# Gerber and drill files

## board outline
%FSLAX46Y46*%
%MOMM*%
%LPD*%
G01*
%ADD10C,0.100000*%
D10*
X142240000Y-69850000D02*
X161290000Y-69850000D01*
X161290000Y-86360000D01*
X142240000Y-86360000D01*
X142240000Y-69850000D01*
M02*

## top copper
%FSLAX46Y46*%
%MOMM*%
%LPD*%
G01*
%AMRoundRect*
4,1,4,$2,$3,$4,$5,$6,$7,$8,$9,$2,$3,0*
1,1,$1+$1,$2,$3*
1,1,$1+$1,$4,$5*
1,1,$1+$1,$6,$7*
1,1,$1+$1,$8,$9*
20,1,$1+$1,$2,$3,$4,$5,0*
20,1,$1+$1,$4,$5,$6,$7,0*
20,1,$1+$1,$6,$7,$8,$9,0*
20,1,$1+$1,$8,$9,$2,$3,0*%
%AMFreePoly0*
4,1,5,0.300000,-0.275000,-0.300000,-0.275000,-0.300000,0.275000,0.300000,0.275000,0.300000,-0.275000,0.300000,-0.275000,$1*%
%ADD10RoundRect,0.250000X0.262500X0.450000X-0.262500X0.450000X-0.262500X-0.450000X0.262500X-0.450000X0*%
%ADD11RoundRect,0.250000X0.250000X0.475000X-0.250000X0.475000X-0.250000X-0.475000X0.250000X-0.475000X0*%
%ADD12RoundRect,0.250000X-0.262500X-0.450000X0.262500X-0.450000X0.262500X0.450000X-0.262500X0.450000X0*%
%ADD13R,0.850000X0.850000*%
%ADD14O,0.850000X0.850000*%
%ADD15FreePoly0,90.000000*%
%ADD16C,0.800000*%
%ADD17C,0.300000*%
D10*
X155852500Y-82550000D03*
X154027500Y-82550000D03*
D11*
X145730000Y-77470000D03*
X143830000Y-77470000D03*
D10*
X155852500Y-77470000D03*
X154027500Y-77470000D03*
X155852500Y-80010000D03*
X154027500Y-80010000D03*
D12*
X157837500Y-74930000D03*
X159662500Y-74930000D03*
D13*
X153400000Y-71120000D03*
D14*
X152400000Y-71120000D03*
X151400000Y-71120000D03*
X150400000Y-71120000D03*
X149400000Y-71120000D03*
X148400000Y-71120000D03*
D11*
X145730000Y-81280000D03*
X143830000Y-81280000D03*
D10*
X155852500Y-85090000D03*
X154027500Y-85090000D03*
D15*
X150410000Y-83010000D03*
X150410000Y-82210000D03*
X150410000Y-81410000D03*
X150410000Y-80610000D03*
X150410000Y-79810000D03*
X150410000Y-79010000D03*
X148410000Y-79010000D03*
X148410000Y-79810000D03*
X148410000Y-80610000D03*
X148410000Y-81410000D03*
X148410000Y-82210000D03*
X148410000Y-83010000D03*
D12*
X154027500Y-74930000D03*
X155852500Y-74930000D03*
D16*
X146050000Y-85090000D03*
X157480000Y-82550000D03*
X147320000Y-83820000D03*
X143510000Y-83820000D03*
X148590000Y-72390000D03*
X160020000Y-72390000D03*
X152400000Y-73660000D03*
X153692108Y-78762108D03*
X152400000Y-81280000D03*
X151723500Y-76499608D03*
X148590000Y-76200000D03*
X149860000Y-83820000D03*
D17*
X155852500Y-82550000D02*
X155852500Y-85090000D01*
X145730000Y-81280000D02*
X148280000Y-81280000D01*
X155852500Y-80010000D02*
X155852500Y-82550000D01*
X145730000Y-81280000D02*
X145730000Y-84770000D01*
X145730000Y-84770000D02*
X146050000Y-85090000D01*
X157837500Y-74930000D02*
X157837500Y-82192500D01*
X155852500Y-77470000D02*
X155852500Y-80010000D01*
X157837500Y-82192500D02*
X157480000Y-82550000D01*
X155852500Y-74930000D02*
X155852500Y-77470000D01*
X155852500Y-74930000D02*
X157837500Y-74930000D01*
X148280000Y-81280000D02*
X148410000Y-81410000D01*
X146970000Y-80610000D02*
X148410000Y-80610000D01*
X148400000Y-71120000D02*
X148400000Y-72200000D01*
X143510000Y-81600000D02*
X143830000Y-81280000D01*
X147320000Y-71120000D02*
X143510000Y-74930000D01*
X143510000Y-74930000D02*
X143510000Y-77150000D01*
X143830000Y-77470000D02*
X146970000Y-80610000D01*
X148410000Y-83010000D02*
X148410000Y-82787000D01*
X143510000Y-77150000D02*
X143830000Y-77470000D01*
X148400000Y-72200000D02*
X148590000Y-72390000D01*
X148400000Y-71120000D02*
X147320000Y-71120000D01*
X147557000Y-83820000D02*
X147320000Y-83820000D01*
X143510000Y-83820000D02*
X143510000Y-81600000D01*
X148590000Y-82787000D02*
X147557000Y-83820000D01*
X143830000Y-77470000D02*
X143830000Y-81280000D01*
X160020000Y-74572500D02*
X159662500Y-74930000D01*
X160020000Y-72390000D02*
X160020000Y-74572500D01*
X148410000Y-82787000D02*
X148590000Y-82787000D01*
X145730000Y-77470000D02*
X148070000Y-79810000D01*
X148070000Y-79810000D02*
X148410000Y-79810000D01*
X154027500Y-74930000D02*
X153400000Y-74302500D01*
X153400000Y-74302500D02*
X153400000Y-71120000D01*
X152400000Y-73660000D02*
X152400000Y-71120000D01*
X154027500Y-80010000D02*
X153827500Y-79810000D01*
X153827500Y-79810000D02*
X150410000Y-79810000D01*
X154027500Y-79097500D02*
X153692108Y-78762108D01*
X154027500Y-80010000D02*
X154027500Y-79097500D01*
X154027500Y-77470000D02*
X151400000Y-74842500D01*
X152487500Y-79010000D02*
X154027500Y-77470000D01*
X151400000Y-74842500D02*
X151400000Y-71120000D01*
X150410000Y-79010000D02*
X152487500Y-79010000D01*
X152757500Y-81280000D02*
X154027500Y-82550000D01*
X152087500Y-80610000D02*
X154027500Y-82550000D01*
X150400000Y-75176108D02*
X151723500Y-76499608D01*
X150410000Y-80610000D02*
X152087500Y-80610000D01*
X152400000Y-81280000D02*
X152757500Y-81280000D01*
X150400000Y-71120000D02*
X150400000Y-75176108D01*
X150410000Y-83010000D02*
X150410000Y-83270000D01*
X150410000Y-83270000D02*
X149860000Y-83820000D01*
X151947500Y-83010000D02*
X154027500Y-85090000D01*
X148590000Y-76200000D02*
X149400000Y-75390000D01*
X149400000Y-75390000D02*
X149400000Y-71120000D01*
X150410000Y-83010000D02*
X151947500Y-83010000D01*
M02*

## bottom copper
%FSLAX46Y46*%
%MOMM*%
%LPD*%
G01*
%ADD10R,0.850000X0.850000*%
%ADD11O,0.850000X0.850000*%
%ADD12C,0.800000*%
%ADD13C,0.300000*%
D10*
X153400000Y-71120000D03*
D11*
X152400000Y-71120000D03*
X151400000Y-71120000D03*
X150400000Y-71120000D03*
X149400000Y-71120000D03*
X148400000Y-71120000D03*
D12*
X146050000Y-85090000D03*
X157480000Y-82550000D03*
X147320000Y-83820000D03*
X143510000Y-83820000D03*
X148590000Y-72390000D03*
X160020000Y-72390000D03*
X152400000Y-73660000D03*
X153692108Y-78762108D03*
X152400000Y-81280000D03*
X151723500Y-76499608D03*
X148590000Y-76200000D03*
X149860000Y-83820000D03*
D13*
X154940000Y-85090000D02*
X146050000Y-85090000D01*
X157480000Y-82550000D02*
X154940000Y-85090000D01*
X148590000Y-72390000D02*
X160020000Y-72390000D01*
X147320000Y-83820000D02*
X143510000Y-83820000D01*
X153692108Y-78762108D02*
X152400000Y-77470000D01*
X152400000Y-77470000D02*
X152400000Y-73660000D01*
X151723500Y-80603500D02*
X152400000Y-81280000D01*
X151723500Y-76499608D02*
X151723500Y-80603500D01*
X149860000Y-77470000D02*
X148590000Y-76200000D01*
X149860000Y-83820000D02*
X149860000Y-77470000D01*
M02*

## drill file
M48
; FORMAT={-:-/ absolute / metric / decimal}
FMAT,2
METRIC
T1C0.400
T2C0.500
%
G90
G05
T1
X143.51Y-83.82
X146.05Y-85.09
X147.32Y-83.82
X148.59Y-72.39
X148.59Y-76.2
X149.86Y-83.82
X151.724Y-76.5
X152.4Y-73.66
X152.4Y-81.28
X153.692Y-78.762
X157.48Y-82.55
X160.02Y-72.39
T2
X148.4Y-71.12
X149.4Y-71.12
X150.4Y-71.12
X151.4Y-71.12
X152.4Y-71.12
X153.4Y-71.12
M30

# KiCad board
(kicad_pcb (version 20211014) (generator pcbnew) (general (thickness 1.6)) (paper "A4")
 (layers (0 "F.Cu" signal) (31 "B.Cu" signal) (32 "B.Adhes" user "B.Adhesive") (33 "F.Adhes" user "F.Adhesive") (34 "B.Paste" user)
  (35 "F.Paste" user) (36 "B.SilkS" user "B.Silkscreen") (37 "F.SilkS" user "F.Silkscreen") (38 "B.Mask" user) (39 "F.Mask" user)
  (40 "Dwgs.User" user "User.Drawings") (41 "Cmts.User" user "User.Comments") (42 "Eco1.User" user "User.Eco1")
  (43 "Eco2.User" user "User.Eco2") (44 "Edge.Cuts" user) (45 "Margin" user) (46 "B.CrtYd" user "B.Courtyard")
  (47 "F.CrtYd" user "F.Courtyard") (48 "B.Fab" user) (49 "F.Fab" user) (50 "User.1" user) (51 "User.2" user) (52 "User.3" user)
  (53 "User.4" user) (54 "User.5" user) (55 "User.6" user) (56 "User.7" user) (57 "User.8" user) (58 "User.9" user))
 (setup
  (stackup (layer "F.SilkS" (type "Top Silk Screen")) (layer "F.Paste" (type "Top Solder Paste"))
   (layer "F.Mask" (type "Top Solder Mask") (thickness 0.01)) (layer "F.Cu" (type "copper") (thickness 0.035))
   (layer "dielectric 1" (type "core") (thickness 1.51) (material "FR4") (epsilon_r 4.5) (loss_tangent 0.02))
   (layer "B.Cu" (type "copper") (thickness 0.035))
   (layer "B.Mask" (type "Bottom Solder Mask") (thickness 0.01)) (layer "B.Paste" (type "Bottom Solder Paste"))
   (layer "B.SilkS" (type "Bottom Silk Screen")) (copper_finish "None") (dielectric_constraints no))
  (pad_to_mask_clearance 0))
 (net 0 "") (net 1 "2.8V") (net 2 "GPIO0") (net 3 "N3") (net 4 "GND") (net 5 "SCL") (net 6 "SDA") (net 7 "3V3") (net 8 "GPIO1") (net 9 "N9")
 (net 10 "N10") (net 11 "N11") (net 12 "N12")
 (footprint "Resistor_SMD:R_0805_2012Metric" (layer "F.Cu") (at 154.94 82.55 180)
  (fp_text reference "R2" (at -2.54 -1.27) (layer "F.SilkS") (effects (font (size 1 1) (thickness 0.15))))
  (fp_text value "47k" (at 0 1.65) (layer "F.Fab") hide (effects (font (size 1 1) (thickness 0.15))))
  (pad "1" smd roundrect (at -0.9125 0 180) (size 1.025 1.4) (layers "F.Cu" "F.Paste" "F.Mask") (roundrect_rratio 0.243902) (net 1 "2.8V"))
  (pad "2" smd roundrect (at 0.9125 0 180) (size 1.025 1.4) (layers "F.Cu" "F.Paste" "F.Mask") (roundrect_rratio 0.243902) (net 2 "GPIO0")))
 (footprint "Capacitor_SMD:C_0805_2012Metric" (layer "F.Cu") (at 144.78 77.47 180)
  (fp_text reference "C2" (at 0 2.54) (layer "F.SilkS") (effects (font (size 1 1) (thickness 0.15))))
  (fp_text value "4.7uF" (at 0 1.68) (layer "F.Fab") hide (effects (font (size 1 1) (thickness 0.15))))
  (pad "1" smd roundrect (at -0.95 0 180) (size 1 1.45) (layers "F.Cu" "F.Paste" "F.Mask") (roundrect_rratio 0.25) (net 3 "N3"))
  (pad "2" smd roundrect (at 0.95 0 180) (size 1 1.45) (layers "F.Cu" "F.Paste" "F.Mask") (roundrect_rratio 0.25) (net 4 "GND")))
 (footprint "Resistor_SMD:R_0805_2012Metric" (layer "F.Cu") (at 154.94 77.47 180)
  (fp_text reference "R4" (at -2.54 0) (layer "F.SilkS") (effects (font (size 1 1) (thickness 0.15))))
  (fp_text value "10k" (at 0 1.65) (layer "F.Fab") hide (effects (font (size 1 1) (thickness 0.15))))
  (pad "1" smd roundrect (at -0.9125 0 180) (size 1.025 1.4) (layers "F.Cu" "F.Paste" "F.Mask") (roundrect_rratio 0.243902) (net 1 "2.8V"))
  (pad "2" smd roundrect (at 0.9125 0 180) (size 1.025 1.4) (layers "F.Cu" "F.Paste" "F.Mask") (roundrect_rratio 0.243902) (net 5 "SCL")))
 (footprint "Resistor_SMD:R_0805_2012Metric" (layer "F.Cu") (at 154.94 80.01 180)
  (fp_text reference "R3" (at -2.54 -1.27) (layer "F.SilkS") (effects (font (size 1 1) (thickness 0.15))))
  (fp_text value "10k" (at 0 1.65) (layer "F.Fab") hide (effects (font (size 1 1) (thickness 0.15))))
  (pad "1" smd roundrect (at -0.9125 0 180) (size 1.025 1.4) (layers "F.Cu" "F.Paste" "F.Mask") (roundrect_rratio 0.243902) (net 1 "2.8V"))
  (pad "2" smd roundrect (at 0.9125 0 180) (size 1.025 1.4) (layers "F.Cu" "F.Paste" "F.Mask") (roundrect_rratio 0.243902) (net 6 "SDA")))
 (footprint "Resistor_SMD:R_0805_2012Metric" (layer "F.Cu") (at 158.75 74.93)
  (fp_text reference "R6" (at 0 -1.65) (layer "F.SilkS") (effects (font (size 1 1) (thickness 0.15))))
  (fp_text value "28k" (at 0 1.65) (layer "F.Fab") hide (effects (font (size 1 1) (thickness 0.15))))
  (pad "1" smd roundrect (at -0.9125 0) (size 1.025 1.4) (layers "F.Cu" "F.Paste" "F.Mask") (roundrect_rratio 0.243902) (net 1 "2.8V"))
  (pad "2" smd roundrect (at 0.9125 0) (size 1.025 1.4) (layers "F.Cu" "F.Paste" "F.Mask") (roundrect_rratio 0.243902) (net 4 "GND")))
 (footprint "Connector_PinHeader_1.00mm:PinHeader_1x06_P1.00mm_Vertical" (layer "F.Cu") (at 153.4 71.12 -90)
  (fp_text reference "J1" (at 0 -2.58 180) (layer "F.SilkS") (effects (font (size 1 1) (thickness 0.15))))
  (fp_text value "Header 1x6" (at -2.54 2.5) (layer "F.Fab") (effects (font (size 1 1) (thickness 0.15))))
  (pad "1" thru_hole rect (at 0 0 270) (size 0.85 0.85) (drill 0.5) (layers *.Cu *.Mask) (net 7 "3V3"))
  (pad "2" thru_hole oval (at 0 1 270) (size 0.85 0.85) (drill 0.5) (layers *.Cu *.Mask) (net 6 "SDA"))
  (pad "3" thru_hole oval (at 0 2 270) (size 0.85 0.85) (drill 0.5) (layers *.Cu *.Mask) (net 5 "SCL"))
  (pad "4" thru_hole oval (at 0 3 270) (size 0.85 0.85) (drill 0.5) (layers *.Cu *.Mask) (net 2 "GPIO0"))
  (pad "5" thru_hole oval (at 0 4 270) (size 0.85 0.85) (drill 0.5) (layers *.Cu *.Mask) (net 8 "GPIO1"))
  (pad "6" thru_hole oval (at 0 5 270) (size 0.85 0.85) (drill 0.5) (layers *.Cu *.Mask) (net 4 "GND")))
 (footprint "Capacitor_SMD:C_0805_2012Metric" (layer "F.Cu") (at 144.78 81.28 180)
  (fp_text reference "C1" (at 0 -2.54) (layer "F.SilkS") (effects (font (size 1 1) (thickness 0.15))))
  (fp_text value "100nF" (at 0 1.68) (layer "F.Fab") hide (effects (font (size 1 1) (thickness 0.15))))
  (pad "1" smd roundrect (at -0.95 0 180) (size 1 1.45) (layers "F.Cu" "F.Paste" "F.Mask") (roundrect_rratio 0.25) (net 1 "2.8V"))
  (pad "2" smd roundrect (at 0.95 0 180) (size 1 1.45) (layers "F.Cu" "F.Paste" "F.Mask") (roundrect_rratio 0.25) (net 4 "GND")))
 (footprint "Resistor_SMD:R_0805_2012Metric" (layer "F.Cu") (at 154.94 85.09 180)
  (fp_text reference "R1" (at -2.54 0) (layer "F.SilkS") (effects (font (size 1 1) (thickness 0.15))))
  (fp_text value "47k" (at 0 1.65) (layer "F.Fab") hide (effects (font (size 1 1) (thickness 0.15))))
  (pad "1" smd roundrect (at -0.9125 0 180) (size 1.025 1.4) (layers "F.Cu" "F.Paste" "F.Mask") (roundrect_rratio 0.243902) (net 1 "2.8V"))
  (pad "2" smd roundrect (at 0.9125 0 180) (size 1.025 1.4) (layers "F.Cu" "F.Paste" "F.Mask") (roundrect_rratio 0.243902) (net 8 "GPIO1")))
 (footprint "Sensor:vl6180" (layer "F.Cu") (at 149.86 80.01 180)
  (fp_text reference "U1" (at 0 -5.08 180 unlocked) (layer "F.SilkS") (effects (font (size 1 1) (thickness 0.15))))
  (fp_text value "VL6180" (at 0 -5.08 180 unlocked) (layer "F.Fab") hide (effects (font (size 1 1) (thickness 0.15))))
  (pad "1" smd custom (at -0.55 -3 90) (size 0.6 0.55) (layers "F.Cu" "F.Paste" "F.Mask") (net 8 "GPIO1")
   (options (clearance outline) (anchor rect)) (primitives))
  (pad "2" smd custom (at -0.55 -2.2 90) (size 0.6 0.55) (layers "F.Cu" "F.Paste" "F.Mask") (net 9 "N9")
   (options (clearance outline) (anchor rect)) (primitives))
  (pad "3" smd custom (at -0.55 -1.4 90) (size 0.6 0.55) (layers "F.Cu" "F.Paste" "F.Mask") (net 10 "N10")
   (options (clearance outline) (anchor rect)) (primitives))
  (pad "4" smd custom (at -0.55 -0.6 90) (size 0.6 0.55) (layers "F.Cu" "F.Paste" "F.Mask") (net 2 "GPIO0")
   (options (clearance outline) (anchor rect)) (primitives))
  (pad "5" smd custom (at -0.55 0.2 90) (size 0.6 0.55) (layers "F.Cu" "F.Paste" "F.Mask") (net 6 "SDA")
   (options (clearance outline) (anchor rect)) (primitives))
  (pad "6" smd custom (at -0.55 1 90) (size 0.6 0.55) (layers "F.Cu" "F.Paste" "F.Mask") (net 5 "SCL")
   (options (clearance outline) (anchor rect)) (primitives))
  (pad "7" smd custom (at 1.45 1 90) (size 0.6 0.55) (layers "F.Cu" "F.Paste" "F.Mask") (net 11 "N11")
   (options (clearance outline) (anchor rect)) (primitives))
  (pad "8" smd custom (at 1.45 0.2 90) (size 0.6 0.55) (layers "F.Cu" "F.Paste" "F.Mask") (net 3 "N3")
   (options (clearance outline) (anchor rect)) (primitives))
  (pad "9" smd custom (at 1.45 -0.6 90) (size 0.6 0.55) (layers "F.Cu" "F.Paste" "F.Mask") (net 4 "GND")
   (options (clearance outline) (anchor rect)) (primitives))
  (pad "10" smd custom (at 1.45 -1.4 90) (size 0.6 0.55) (layers "F.Cu" "F.Paste" "F.Mask") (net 1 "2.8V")
   (options (clearance outline) (anchor rect)) (primitives))
  (pad "11" smd custom (at 1.45 -2.2 90) (size 0.6 0.55) (layers "F.Cu" "F.Paste" "F.Mask") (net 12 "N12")
   (options (clearance outline) (anchor rect)) (primitives))
  (pad "12" smd custom (at 1.45 -3 90) (size 0.6 0.55) (layers "F.Cu" "F.Paste" "F.Mask") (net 4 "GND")
   (options (clearance outline) (anchor rect)) (primitives)))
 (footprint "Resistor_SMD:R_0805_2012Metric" (layer "F.Cu") (at 154.94 74.93)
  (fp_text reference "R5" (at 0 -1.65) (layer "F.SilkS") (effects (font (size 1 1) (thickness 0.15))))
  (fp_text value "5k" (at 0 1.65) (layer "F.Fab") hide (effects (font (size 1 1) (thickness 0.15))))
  (pad "1" smd roundrect (at -0.9125 0) (size 1.025 1.4) (layers "F.Cu" "F.Paste" "F.Mask") (roundrect_rratio 0.243902) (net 7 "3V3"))
  (pad "2" smd roundrect (at 0.9125 0) (size 1.025 1.4) (layers "F.Cu" "F.Paste" "F.Mask") (roundrect_rratio 0.243902) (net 1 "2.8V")))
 (gr_rect (start 142.24 69.85) (end 161.29 86.36) (layer "Edge.Cuts") (width 0.1) (fill none))
 (segment (start 155.8525 82.55) (end 155.8525 85.09) (width 0.3) (layer "F.Cu") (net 1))
 (segment (start 145.73 81.28) (end 148.28 81.28) (width 0.3) (layer "F.Cu") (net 1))
 (segment (start 155.8525 80.01) (end 155.8525 82.55) (width 0.3) (layer "F.Cu") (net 1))
 (segment (start 145.73 81.28) (end 145.73 84.77) (width 0.3) (layer "F.Cu") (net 1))
 (segment (start 145.73 84.77) (end 146.05 85.09) (width 0.3) (layer "F.Cu") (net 1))
 (segment (start 157.8375 74.93) (end 157.8375 82.1925) (width 0.3) (layer "F.Cu") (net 1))
 (segment (start 155.8525 77.47) (end 155.8525 80.01) (width 0.3) (layer "F.Cu") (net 1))
 (segment (start 157.8375 82.1925) (end 157.48 82.55) (width 0.3) (layer "F.Cu") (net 1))
 (segment (start 155.8525 74.93) (end 155.8525 77.47) (width 0.3) (layer "F.Cu") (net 1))
 (segment (start 155.8525 74.93) (end 157.8375 74.93) (width 0.3) (layer "F.Cu") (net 1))
 (segment (start 148.28 81.28) (end 148.41 81.41) (width 0.3) (layer "F.Cu") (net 1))
 (via (at 146.05 85.09) (size 0.8) (drill 0.4) (layers "F.Cu" "B.Cu") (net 1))
 (via (at 157.48 82.55) (size 0.8) (drill 0.4) (layers "F.Cu" "B.Cu") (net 1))
 (segment (start 154.94 85.09) (end 146.05 85.09) (width 0.3) (layer "B.Cu") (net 1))
 (segment (start 157.48 82.55) (end 154.94 85.09) (width 0.3) (layer "B.Cu") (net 1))
 (segment (start 146.97 80.61) (end 148.41 80.61) (width 0.3) (layer "F.Cu") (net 4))
 (segment (start 148.4 71.12) (end 148.4 72.2) (width 0.3) (layer "F.Cu") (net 4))
 (segment (start 143.51 81.6) (end 143.83 81.28) (width 0.3) (layer "F.Cu") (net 4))
 (segment (start 147.32 71.12) (end 143.51 74.93) (width 0.3) (layer "F.Cu") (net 4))
 (segment (start 143.51 74.93) (end 143.51 77.15) (width 0.3) (layer "F.Cu") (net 4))
 (segment (start 143.83 77.47) (end 146.97 80.61) (width 0.3) (layer "F.Cu") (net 4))
 (segment (start 148.41 83.01) (end 148.41 82.787) (width 0.3) (layer "F.Cu") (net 4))
 (segment (start 143.51 77.15) (end 143.83 77.47) (width 0.3) (layer "F.Cu") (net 4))
 (segment (start 148.4 72.2) (end 148.59 72.39) (width 0.3) (layer "F.Cu") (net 4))
 (segment (start 148.4 71.12) (end 147.32 71.12) (width 0.3) (layer "F.Cu") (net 4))
 (segment (start 147.557 83.82) (end 147.32 83.82) (width 0.3) (layer "F.Cu") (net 4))
 (segment (start 143.51 83.82) (end 143.51 81.6) (width 0.3) (layer "F.Cu") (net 4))
 (segment (start 148.59 82.787) (end 147.557 83.82) (width 0.3) (layer "F.Cu") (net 4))
 (segment (start 143.83 77.47) (end 143.83 81.28) (width 0.3) (layer "F.Cu") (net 4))
 (segment (start 160.02 74.5725) (end 159.6625 74.93) (width 0.3) (layer "F.Cu") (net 4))
 (segment (start 160.02 72.39) (end 160.02 74.5725) (width 0.3) (layer "F.Cu") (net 4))
 (segment (start 148.41 82.787) (end 148.59 82.787) (width 0.3) (layer "F.Cu") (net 4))
 (via (at 147.32 83.82) (size 0.8) (drill 0.4) (layers "F.Cu" "B.Cu") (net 4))
 (via (at 143.51 83.82) (size 0.8) (drill 0.4) (layers "F.Cu" "B.Cu") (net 4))
 (via (at 148.59 72.39) (size 0.8) (drill 0.4) (layers "F.Cu" "B.Cu") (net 4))
 (via (at 160.02 72.39) (size 0.8) (drill 0.4) (layers "F.Cu" "B.Cu") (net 4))
 (segment (start 148.59 72.39) (end 160.02 72.39) (width 0.3) (layer "B.Cu") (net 4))
 (segment (start 147.32 83.82) (end 143.51 83.82) (width 0.3) (layer "B.Cu") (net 4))
 (segment (start 145.73 77.47) (end 148.07 79.81) (width 0.3) (layer "F.Cu") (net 3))
 (segment (start 148.07 79.81) (end 148.41 79.81) (width 0.3) (layer "F.Cu") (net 3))
 (segment (start 154.0275 74.93) (end 153.4 74.3025) (width 0.3) (layer "F.Cu") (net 7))
 (segment (start 153.4 74.3025) (end 153.4 71.12) (width 0.3) (layer "F.Cu") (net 7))
 (segment (start 152.4 73.66) (end 152.4 71.12) (width 0.3) (layer "F.Cu") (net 6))
 (segment (start 154.0275 80.01) (end 153.8275 79.81) (width 0.3) (layer "F.Cu") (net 6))
 (segment (start 153.8275 79.81) (end 150.41 79.81) (width 0.3) (layer "F.Cu") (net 6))
 (segment (start 154.0275 79.0975) (end 153.692108 78.762108) (width 0.3) (layer "F.Cu") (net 6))
 (segment (start 154.0275 80.01) (end 154.0275 79.0975) (width 0.3) (layer "F.Cu") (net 6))
 (via (at 152.4 73.66) (size 0.8) (drill 0.4) (layers "F.Cu" "B.Cu") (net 6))
 (via (at 153.692108 78.762108) (size 0.8) (drill 0.4) (layers "F.Cu" "B.Cu") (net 6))
 (segment (start 153.692108 78.762108) (end 152.4 77.47) (width 0.3) (layer "B.Cu") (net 6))
 (segment (start 152.4 77.47) (end 152.4 73.66) (width 0.3) (layer "B.Cu") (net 6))
 (segment (start 154.0275 77.47) (end 151.4 74.8425) (width 0.3) (layer "F.Cu") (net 5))
 (segment (start 152.4875 79.01) (end 154.0275 77.47) (width 0.3) (layer "F.Cu") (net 5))
 (segment (start 151.4 74.8425) (end 151.4 71.12) (width 0.3) (layer "F.Cu") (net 5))
 (segment (start 150.41 79.01) (end 152.4875 79.01) (width 0.3) (layer "F.Cu") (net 5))
 (segment (start 152.7575 81.28) (end 154.0275 82.55) (width 0.3) (layer "F.Cu") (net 2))
 (segment (start 152.0875 80.61) (end 154.0275 82.55) (width 0.3) (layer "F.Cu") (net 2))
 (segment (start 150.4 75.176108) (end 151.7235 76.499608) (width 0.3) (layer "F.Cu") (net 2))
 (segment (start 150.41 80.61) (end 152.0875 80.61) (width 0.3) (layer "F.Cu") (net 2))
 (segment (start 152.4 81.28) (end 152.7575 81.28) (width 0.3) (layer "F.Cu") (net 2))
 (segment (start 150.4 71.12) (end 150.4 75.176108) (width 0.3) (layer "F.Cu") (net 2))
 (via (at 152.4 81.28) (size 0.8) (drill 0.4) (layers "F.Cu" "B.Cu") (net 2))
 (via (at 151.7235 76.499608) (size 0.8) (drill 0.4) (layers "F.Cu" "B.Cu") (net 2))
 (segment (start 151.7235 80.6035) (end 152.4 81.28) (width 0.3) (layer "B.Cu") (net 2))
 (segment (start 151.7235 76.499608) (end 151.7235 80.6035) (width 0.3) (layer "B.Cu") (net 2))
 (segment (start 150.41 83.01) (end 150.41 83.27) (width 0.3) (layer "F.Cu") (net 8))
 (segment (start 150.41 83.27) (end 149.86 83.82) (width 0.3) (layer "F.Cu") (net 8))
 (segment (start 151.9475 83.01) (end 154.0275 85.09) (width 0.3) (layer "F.Cu") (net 8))
 (segment (start 148.59 76.2) (end 149.4 75.39) (width 0.3) (layer "F.Cu") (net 8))
 (segment (start 149.4 75.39) (end 149.4 71.12) (width 0.3) (layer "F.Cu") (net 8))
 (segment (start 150.41 83.01) (end 151.9475 83.01) (width 0.3) (layer "F.Cu") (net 8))
 (via (at 148.59 76.2) (size 0.8) (drill 0.4) (layers "F.Cu" "B.Cu") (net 8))
 (via (at 149.86 83.82) (size 0.8) (drill 0.4) (layers "F.Cu" "B.Cu") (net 8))
 (segment (start 149.86 77.47) (end 148.59 76.2) (width 0.3) (layer "B.Cu") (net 8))
 (segment (start 149.86 83.82) (end 149.86 77.47) (width 0.3) (layer "B.Cu") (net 8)))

